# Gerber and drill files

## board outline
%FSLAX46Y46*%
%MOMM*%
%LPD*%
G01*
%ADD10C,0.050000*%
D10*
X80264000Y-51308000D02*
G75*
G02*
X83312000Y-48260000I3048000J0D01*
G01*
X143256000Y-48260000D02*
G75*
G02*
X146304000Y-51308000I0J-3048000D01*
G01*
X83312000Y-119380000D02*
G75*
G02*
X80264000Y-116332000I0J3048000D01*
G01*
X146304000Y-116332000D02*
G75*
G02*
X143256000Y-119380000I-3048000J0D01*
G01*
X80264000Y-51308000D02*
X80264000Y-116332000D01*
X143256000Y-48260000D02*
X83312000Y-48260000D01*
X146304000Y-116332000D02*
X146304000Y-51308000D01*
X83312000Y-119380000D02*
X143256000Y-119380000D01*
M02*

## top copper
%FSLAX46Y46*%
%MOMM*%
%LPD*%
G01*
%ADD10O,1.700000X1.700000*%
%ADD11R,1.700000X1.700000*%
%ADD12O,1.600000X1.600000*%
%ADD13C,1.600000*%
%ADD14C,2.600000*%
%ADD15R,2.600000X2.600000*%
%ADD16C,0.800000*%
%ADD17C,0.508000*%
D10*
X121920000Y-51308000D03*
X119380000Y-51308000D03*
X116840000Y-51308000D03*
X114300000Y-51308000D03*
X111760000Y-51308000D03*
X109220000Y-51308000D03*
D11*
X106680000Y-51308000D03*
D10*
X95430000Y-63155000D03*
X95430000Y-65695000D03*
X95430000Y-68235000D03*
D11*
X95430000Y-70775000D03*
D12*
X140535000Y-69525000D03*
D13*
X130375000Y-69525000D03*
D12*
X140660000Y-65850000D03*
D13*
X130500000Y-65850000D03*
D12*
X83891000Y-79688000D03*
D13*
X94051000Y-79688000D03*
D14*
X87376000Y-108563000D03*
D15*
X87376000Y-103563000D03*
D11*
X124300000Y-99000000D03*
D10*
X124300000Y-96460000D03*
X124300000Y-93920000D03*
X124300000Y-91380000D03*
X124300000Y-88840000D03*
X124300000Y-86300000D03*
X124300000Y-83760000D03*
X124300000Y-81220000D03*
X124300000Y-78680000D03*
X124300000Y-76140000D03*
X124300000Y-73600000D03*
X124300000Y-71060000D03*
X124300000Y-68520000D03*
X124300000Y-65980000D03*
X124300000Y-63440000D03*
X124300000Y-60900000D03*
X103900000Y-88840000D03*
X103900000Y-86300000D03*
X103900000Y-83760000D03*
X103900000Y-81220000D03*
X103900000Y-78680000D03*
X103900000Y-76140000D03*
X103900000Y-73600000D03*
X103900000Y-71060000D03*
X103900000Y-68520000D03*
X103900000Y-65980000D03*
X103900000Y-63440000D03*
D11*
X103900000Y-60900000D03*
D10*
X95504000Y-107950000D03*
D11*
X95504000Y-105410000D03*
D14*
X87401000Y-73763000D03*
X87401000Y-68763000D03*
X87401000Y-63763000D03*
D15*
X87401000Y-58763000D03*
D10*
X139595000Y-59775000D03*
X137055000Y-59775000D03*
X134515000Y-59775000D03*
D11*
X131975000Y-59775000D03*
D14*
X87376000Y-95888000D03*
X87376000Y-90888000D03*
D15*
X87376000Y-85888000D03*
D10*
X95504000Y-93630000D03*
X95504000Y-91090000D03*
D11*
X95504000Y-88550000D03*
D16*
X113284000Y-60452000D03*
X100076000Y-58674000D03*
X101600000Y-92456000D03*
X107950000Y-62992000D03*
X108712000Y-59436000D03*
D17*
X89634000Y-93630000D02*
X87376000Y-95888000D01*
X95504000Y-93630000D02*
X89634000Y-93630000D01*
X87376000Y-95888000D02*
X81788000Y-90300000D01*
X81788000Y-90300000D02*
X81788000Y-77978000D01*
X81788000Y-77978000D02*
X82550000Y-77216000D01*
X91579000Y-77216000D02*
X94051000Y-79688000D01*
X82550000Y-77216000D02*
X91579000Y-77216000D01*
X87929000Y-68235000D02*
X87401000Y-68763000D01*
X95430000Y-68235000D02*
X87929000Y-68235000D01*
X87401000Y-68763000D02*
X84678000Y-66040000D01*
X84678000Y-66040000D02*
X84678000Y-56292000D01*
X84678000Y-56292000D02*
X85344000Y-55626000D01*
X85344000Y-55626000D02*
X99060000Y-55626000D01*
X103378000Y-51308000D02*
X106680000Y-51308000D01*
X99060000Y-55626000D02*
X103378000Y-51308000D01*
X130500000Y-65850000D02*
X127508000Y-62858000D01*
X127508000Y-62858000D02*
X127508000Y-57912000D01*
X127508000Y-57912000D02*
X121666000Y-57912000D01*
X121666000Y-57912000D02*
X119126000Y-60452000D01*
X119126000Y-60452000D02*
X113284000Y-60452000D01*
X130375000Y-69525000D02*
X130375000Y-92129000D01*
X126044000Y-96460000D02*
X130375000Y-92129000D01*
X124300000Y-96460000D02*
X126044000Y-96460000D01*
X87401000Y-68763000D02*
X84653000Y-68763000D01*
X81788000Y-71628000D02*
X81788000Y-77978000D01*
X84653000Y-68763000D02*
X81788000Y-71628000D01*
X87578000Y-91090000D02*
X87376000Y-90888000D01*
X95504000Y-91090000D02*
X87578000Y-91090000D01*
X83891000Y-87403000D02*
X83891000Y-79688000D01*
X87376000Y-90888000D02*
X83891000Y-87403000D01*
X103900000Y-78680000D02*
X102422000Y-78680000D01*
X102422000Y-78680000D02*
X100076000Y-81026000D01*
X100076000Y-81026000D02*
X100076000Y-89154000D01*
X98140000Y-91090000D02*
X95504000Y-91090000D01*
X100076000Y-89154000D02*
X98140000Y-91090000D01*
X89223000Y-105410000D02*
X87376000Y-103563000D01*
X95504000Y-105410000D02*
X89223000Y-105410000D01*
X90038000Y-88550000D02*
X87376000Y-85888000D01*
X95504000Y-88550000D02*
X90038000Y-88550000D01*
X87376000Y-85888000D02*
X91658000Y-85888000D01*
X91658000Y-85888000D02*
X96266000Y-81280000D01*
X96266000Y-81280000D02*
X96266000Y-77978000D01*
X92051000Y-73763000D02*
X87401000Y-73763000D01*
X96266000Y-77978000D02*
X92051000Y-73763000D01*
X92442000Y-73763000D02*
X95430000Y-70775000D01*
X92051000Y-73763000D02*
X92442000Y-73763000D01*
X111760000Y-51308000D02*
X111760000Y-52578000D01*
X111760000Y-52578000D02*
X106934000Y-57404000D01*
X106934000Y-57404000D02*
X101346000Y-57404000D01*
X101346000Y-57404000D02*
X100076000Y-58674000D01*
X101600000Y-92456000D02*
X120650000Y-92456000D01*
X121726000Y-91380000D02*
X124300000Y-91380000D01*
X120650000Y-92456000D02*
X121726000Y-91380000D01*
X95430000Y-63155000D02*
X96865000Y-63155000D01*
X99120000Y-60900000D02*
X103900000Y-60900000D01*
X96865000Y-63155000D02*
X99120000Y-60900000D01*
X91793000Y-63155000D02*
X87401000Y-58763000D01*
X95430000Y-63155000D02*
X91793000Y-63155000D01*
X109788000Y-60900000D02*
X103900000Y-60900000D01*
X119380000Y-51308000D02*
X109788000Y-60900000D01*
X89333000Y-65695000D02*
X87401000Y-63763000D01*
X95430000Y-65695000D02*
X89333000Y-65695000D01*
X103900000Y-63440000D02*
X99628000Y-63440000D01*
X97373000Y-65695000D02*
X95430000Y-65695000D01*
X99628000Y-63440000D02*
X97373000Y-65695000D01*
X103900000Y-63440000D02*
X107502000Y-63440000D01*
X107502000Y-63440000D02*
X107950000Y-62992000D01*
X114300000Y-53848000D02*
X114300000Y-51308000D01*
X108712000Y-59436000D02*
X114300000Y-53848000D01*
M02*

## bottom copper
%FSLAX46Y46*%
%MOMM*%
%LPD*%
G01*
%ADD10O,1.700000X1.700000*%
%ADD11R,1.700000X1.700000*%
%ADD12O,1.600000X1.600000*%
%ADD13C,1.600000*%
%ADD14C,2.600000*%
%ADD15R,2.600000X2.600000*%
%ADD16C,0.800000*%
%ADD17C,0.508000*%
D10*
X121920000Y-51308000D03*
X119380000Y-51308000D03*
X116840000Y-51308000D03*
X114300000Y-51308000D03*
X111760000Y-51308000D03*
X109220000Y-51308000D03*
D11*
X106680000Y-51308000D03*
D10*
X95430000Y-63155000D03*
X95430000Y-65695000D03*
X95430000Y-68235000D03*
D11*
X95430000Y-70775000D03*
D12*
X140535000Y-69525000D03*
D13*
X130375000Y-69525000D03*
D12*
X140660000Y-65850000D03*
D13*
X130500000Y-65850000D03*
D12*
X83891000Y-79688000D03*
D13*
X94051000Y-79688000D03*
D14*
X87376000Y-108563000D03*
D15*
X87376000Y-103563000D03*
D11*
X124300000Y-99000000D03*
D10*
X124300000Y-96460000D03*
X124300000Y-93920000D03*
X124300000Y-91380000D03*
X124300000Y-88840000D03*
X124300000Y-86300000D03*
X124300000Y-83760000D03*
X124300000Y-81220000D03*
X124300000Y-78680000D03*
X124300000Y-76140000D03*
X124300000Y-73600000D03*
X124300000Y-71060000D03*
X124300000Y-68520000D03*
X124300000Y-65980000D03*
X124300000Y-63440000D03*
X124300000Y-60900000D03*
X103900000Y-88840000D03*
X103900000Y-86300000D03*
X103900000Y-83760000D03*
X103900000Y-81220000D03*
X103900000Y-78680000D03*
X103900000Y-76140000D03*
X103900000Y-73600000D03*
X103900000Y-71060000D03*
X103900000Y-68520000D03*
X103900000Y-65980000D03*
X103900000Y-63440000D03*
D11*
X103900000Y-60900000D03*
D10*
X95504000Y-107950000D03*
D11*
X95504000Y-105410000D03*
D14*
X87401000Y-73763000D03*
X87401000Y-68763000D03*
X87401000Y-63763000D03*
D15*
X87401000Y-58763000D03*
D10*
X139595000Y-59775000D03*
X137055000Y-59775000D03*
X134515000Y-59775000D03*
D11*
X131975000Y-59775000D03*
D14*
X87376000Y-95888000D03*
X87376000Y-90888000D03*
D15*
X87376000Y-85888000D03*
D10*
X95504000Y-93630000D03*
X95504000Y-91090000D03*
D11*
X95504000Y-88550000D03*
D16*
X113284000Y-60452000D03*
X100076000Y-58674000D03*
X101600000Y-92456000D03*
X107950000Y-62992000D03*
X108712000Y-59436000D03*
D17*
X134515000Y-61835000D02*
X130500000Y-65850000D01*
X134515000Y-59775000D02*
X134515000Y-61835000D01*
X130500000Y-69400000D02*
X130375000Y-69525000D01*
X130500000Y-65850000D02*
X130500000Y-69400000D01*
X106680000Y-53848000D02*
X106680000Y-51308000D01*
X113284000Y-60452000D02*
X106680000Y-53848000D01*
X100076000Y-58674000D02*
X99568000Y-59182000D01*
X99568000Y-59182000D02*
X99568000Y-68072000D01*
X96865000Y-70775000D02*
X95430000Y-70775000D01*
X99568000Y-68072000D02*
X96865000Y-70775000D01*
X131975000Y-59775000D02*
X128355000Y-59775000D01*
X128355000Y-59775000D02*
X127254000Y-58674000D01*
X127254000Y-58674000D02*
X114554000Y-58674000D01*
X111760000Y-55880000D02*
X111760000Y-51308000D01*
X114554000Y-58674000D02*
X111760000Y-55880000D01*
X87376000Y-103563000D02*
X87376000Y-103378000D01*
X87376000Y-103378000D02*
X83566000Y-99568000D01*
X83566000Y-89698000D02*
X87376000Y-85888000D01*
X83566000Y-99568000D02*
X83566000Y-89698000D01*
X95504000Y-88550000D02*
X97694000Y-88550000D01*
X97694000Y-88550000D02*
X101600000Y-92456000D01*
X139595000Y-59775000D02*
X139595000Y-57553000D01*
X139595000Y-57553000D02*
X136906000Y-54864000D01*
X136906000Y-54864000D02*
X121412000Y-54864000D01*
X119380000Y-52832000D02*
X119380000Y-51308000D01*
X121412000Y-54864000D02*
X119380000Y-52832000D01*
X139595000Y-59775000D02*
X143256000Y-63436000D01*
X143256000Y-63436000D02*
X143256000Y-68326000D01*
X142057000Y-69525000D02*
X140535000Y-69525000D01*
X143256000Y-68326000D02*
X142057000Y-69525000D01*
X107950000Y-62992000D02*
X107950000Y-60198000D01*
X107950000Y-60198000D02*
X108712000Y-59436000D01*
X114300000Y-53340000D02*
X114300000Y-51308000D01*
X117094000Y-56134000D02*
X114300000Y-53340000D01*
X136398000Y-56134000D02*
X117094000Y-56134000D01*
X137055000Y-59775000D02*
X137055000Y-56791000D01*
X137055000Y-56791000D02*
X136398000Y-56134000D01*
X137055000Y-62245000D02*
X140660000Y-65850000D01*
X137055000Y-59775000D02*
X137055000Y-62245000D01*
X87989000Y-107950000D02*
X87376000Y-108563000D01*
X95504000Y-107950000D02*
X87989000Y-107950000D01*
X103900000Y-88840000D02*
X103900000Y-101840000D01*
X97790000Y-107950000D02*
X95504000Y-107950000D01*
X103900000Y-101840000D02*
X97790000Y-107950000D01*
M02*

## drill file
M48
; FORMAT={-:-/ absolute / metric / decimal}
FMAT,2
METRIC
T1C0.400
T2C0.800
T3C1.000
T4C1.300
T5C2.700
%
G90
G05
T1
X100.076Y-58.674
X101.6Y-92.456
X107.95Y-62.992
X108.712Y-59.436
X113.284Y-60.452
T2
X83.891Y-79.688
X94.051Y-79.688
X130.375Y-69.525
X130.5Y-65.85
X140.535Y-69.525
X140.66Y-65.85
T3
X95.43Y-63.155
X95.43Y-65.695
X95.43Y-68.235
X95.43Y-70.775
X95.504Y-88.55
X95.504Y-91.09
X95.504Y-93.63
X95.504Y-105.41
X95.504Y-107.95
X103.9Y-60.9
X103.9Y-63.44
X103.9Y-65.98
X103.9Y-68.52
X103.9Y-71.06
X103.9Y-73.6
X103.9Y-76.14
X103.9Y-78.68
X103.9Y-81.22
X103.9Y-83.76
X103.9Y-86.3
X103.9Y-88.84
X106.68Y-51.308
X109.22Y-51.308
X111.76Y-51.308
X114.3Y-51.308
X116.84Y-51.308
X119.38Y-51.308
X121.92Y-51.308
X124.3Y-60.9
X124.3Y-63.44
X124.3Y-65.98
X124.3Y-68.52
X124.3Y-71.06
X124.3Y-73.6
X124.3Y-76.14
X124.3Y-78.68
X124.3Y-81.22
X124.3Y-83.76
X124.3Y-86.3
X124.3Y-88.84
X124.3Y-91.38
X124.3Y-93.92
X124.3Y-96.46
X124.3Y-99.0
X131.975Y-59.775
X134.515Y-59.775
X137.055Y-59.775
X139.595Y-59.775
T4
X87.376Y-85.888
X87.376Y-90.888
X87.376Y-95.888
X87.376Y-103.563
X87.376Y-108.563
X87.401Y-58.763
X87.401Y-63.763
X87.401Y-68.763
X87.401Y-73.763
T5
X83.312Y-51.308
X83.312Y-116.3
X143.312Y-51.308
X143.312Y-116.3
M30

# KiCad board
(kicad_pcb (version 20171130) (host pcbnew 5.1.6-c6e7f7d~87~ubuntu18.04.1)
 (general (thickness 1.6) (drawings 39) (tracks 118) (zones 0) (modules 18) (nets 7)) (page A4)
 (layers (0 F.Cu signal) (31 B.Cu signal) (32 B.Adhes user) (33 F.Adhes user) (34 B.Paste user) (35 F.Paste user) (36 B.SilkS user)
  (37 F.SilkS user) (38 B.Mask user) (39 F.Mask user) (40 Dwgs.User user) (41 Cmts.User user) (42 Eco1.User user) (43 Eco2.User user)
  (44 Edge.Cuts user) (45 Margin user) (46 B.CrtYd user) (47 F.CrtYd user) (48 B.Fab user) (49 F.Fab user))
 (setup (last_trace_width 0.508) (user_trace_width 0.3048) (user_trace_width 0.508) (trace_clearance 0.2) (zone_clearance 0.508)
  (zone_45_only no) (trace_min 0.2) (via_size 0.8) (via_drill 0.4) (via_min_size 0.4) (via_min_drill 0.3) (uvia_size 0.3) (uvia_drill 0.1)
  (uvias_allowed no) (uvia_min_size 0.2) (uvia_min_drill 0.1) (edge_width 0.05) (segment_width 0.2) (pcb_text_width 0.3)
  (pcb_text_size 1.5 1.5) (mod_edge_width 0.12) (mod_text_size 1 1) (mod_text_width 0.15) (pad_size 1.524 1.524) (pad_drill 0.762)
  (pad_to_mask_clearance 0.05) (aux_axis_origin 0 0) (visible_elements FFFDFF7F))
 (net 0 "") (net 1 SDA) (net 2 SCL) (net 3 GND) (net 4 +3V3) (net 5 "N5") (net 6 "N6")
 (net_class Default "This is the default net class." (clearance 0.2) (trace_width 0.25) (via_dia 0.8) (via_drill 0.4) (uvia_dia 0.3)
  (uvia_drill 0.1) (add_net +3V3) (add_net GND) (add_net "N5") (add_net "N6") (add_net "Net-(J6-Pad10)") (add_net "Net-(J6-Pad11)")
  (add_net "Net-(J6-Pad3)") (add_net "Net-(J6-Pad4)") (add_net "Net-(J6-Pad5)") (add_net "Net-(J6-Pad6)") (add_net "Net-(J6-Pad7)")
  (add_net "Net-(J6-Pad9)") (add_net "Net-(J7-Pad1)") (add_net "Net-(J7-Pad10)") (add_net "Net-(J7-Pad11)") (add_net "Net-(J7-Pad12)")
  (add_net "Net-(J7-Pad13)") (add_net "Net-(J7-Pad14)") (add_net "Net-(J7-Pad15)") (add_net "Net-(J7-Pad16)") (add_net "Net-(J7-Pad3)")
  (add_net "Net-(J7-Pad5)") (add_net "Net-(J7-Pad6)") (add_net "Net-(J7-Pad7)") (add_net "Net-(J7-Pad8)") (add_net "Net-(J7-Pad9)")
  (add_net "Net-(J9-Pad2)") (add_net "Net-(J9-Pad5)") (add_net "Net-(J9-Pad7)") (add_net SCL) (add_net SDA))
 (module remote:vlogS (layer F.Cu) (at 136.652 107.442)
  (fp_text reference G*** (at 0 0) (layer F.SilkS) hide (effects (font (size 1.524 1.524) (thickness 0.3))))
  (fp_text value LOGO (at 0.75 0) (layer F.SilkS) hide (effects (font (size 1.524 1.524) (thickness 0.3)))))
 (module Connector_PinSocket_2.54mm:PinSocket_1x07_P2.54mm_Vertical (layer F.Cu) (at 106.68 51.308 90)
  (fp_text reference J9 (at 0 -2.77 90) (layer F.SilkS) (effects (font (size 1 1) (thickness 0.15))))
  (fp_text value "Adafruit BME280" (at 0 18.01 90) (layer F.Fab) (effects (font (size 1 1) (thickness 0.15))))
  (pad 7 thru_hole oval (at 0 15.24 90) (size 1.7 1.7) (drill 1) (layers *.Cu *.Mask))
  (pad 6 thru_hole oval (at 0 12.7 90) (size 1.7 1.7) (drill 1) (layers *.Cu *.Mask) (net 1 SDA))
  (pad 5 thru_hole oval (at 0 10.16 90) (size 1.7 1.7) (drill 1) (layers *.Cu *.Mask))
  (pad 4 thru_hole oval (at 0 7.62 90) (size 1.7 1.7) (drill 1) (layers *.Cu *.Mask) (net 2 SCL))
  (pad 3 thru_hole oval (at 0 5.08 90) (size 1.7 1.7) (drill 1) (layers *.Cu *.Mask) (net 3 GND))
  (pad 2 thru_hole oval (at 0 2.54 90) (size 1.7 1.7) (drill 1) (layers *.Cu *.Mask))
  (pad 1 thru_hole rect (at 0 0 90) (size 1.7 1.7) (drill 1) (layers *.Cu *.Mask) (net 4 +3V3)))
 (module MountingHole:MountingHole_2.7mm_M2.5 (layer F.Cu) (at 143.312 116.3)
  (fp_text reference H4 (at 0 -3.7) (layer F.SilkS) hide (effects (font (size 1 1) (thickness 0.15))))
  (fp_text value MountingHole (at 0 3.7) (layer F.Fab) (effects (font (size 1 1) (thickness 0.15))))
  (pad 1 np_thru_hole circle (at 0 0) (size 2.7 2.7) (drill 2.7) (layers *.Cu *.Mask)))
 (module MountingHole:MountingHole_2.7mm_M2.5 (layer F.Cu) (at 83.312 116.3)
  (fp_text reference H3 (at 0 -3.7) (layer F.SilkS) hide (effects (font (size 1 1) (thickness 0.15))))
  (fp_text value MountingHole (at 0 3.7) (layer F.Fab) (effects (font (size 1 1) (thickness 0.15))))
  (pad 1 np_thru_hole circle (at 0 0) (size 2.7 2.7) (drill 2.7) (layers *.Cu *.Mask)))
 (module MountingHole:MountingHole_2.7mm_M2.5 (layer F.Cu) (at 143.312 51.308)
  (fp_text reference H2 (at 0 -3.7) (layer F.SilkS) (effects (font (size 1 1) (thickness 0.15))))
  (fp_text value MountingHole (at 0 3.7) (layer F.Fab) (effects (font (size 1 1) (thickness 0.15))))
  (pad 1 np_thru_hole circle (at 0 0) (size 2.7 2.7) (drill 2.7) (layers *.Cu *.Mask)))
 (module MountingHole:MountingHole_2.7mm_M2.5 (layer F.Cu) (at 83.312 51.308)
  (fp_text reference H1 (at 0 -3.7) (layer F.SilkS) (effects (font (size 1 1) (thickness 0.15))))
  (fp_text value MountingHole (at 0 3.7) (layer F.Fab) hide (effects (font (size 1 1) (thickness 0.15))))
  (pad 1 np_thru_hole circle (at 0 0) (size 2.7 2.7) (drill 2.7) (layers *.Cu *.Mask)))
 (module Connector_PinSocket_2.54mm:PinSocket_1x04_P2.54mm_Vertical (layer F.Cu) (at 95.43 70.775 180)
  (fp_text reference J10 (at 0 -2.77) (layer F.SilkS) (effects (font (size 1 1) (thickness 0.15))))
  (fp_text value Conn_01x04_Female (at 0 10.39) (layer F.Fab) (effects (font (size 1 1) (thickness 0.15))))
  (pad 4 thru_hole oval (at 0 7.62 180) (size 1.7 1.7) (drill 1) (layers *.Cu *.Mask) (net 1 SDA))
  (pad 3 thru_hole oval (at 0 5.08 180) (size 1.7 1.7) (drill 1) (layers *.Cu *.Mask) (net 2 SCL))
  (pad 2 thru_hole oval (at 0 2.54 180) (size 1.7 1.7) (drill 1) (layers *.Cu *.Mask) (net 4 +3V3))
  (pad 1 thru_hole rect (at 0 0 180) (size 1.7 1.7) (drill 1) (layers *.Cu *.Mask) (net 3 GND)))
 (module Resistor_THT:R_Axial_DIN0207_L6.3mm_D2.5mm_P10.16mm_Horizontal (layer F.Cu) (at 130.375 69.525)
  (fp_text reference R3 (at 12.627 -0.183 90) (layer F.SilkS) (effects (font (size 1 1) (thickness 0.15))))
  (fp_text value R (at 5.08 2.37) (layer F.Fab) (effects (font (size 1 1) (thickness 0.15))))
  (pad 2 thru_hole oval (at 10.16 0) (size 1.6 1.6) (drill 0.8) (layers *.Cu *.Mask) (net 1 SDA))
  (pad 1 thru_hole circle (at 0 0) (size 1.6 1.6) (drill 0.8) (layers *.Cu *.Mask) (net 4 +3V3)))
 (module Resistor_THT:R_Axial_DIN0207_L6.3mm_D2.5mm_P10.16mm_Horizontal (layer F.Cu) (at 130.5 65.85)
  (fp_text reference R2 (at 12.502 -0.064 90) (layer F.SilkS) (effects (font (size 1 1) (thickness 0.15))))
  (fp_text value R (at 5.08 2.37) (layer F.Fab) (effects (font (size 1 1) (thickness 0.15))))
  (pad 2 thru_hole oval (at 10.16 0) (size 1.6 1.6) (drill 0.8) (layers *.Cu *.Mask) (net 2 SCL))
  (pad 1 thru_hole circle (at 0 0) (size 1.6 1.6) (drill 0.8) (layers *.Cu *.Mask) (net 4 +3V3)))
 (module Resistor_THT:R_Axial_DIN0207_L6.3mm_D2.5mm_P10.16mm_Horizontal (layer F.Cu) (at 94.051 79.688 180)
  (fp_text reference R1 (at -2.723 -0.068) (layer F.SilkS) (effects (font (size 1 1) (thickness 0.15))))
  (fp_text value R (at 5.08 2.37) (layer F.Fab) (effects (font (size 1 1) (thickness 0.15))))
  (pad 2 thru_hole oval (at 10.16 0 180) (size 1.6 1.6) (drill 0.8) (layers *.Cu *.Mask) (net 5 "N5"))
  (pad 1 thru_hole circle (at 0 0 180) (size 1.6 1.6) (drill 0.8) (layers *.Cu *.Mask) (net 4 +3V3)))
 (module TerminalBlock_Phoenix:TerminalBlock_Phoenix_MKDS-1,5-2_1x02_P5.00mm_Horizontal (layer F.Cu) (at 87.376 103.563 270)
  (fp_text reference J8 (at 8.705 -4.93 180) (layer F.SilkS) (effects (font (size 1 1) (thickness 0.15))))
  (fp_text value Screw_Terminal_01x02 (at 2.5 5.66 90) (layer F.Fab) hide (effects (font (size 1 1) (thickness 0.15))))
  (pad 2 thru_hole circle (at 5 0 270) (size 2.6 2.6) (drill 1.3) (layers *.Cu *.Mask) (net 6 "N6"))
  (pad 1 thru_hole rect (at 0 0 270) (size 2.6 2.6) (drill 1.3) (layers *.Cu *.Mask) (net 3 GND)))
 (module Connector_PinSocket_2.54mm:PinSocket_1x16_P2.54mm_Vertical (layer F.Cu) (at 124.3 99 180)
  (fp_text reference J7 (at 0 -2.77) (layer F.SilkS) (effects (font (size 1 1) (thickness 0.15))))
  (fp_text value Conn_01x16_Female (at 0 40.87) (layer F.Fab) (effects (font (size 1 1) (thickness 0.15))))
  (pad 1 thru_hole rect (at 0 0 180) (size 1.7 1.7) (drill 1) (layers *.Cu *.Mask))
  (pad 2 thru_hole oval (at 0 2.54 180) (size 1.7 1.7) (drill 1) (layers *.Cu *.Mask) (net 4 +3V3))
  (pad 3 thru_hole oval (at 0 5.08 180) (size 1.7 1.7) (drill 1) (layers *.Cu *.Mask))
  (pad 4 thru_hole oval (at 0 7.62 180) (size 1.7 1.7) (drill 1) (layers *.Cu *.Mask) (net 3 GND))
  (pad 5 thru_hole oval (at 0 10.16 180) (size 1.7 1.7) (drill 1) (layers *.Cu *.Mask))
  (pad 6 thru_hole oval (at 0 12.7 180) (size 1.7 1.7) (drill 1) (layers *.Cu *.Mask))
  (pad 7 thru_hole oval (at 0 15.24 180) (size 1.7 1.7) (drill 1) (layers *.Cu *.Mask))
  (pad 8 thru_hole oval (at 0 17.78 180) (size 1.7 1.7) (drill 1) (layers *.Cu *.Mask))
  (pad 9 thru_hole oval (at 0 20.32 180) (size 1.7 1.7) (drill 1) (layers *.Cu *.Mask))
  (pad 10 thru_hole oval (at 0 22.86 180) (size 1.7 1.7) (drill 1) (layers *.Cu *.Mask))
  (pad 11 thru_hole oval (at 0 25.4 180) (size 1.7 1.7) (drill 1) (layers *.Cu *.Mask))
  (pad 12 thru_hole oval (at 0 27.94 180) (size 1.7 1.7) (drill 1) (layers *.Cu *.Mask))
  (pad 13 thru_hole oval (at 0 30.48 180) (size 1.7 1.7) (drill 1) (layers *.Cu *.Mask))
  (pad 14 thru_hole oval (at 0 33.02 180) (size 1.7 1.7) (drill 1) (layers *.Cu *.Mask))
  (pad 15 thru_hole oval (at 0 35.56 180) (size 1.7 1.7) (drill 1) (layers *.Cu *.Mask))
  (pad 16 thru_hole oval (at 0 38.1 180) (size 1.7 1.7) (drill 1) (layers *.Cu *.Mask)))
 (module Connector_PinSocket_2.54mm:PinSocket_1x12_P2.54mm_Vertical (layer F.Cu) (at 103.9 60.9)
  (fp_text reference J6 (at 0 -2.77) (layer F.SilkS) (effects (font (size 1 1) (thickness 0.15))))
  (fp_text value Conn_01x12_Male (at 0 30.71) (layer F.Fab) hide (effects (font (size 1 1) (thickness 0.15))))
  (pad 12 thru_hole oval (at 0 27.94) (size 1.7 1.7) (drill 1) (layers *.Cu *.Mask) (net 6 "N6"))
  (pad 11 thru_hole oval (at 0 25.4) (size 1.7 1.7) (drill 1) (layers *.Cu *.Mask))
  (pad 10 thru_hole oval (at 0 22.86) (size 1.7 1.7) (drill 1) (layers *.Cu *.Mask))
  (pad 9 thru_hole oval (at 0 20.32) (size 1.7 1.7) (drill 1) (layers *.Cu *.Mask))
  (pad 8 thru_hole oval (at 0 17.78) (size 1.7 1.7) (drill 1) (layers *.Cu *.Mask) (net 5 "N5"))
  (pad 7 thru_hole oval (at 0 15.24) (size 1.7 1.7) (drill 1) (layers *.Cu *.Mask))
  (pad 6 thru_hole oval (at 0 12.7) (size 1.7 1.7) (drill 1) (layers *.Cu *.Mask))
  (pad 5 thru_hole oval (at 0 10.16) (size 1.7 1.7) (drill 1) (layers *.Cu *.Mask))
  (pad 4 thru_hole oval (at 0 7.62) (size 1.7 1.7) (drill 1) (layers *.Cu *.Mask))
  (pad 3 thru_hole oval (at 0 5.08) (size 1.7 1.7) (drill 1) (layers *.Cu *.Mask))
  (pad 2 thru_hole oval (at 0 2.54) (size 1.7 1.7) (drill 1) (layers *.Cu *.Mask) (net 2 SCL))
  (pad 1 thru_hole rect (at 0 0) (size 1.7 1.7) (drill 1) (layers *.Cu *.Mask) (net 1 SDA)))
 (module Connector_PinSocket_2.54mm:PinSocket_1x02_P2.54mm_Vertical (layer F.Cu) (at 95.504 105.41)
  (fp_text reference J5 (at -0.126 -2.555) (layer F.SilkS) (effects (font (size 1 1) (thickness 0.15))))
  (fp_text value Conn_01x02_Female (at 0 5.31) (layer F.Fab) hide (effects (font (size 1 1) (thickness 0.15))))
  (pad 2 thru_hole oval (at 0 2.54) (size 1.7 1.7) (drill 1) (layers *.Cu *.Mask) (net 6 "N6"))
  (pad 1 thru_hole rect (at 0 0) (size 1.7 1.7) (drill 1) (layers *.Cu *.Mask) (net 3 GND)))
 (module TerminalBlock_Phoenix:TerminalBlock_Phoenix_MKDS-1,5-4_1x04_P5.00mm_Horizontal (layer F.Cu) (at 87.401 58.763 270)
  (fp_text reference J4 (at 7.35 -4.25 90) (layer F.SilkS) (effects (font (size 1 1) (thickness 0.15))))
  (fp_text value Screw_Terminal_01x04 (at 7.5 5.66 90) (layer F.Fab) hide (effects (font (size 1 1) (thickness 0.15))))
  (pad 4 thru_hole circle (at 15 0 270) (size 2.6 2.6) (drill 1.3) (layers *.Cu *.Mask) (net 3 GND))
  (pad 3 thru_hole circle (at 10 0 270) (size 2.6 2.6) (drill 1.3) (layers *.Cu *.Mask) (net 4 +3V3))
  (pad 2 thru_hole circle (at 5 0 270) (size 2.6 2.6) (drill 1.3) (layers *.Cu *.Mask) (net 2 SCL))
  (pad 1 thru_hole rect (at 0 0 270) (size 2.6 2.6) (drill 1.3) (layers *.Cu *.Mask) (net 1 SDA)))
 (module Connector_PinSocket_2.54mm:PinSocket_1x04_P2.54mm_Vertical (layer F.Cu) (at 131.975 59.775 90)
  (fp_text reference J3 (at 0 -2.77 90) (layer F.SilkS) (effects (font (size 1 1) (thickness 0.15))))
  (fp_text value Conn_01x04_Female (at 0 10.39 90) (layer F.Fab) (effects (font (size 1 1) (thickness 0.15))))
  (pad 4 thru_hole oval (at 0 7.62 90) (size 1.7 1.7) (drill 1) (layers *.Cu *.Mask) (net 1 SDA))
  (pad 3 thru_hole oval (at 0 5.08 90) (size 1.7 1.7) (drill 1) (layers *.Cu *.Mask) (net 2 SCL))
  (pad 2 thru_hole oval (at 0 2.54 90) (size 1.7 1.7) (drill 1) (layers *.Cu *.Mask) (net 4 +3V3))
  (pad 1 thru_hole rect (at 0 0 90) (size 1.7 1.7) (drill 1) (layers *.Cu *.Mask) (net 3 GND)))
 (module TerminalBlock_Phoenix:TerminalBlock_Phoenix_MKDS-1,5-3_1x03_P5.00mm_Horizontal (layer F.Cu) (at 87.376 85.888 270)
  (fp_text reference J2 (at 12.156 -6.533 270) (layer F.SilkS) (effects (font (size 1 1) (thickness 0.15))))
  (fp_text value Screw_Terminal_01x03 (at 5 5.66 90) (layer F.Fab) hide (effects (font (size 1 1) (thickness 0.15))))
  (pad 3 thru_hole circle (at 10 0 270) (size 2.6 2.6) (drill 1.3) (layers *.Cu *.Mask) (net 4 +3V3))
  (pad 2 thru_hole circle (at 5 0 270) (size 2.6 2.6) (drill 1.3) (layers *.Cu *.Mask) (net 5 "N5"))
  (pad 1 thru_hole rect (at 0 0 270) (size 2.6 2.6) (drill 1.3) (layers *.Cu *.Mask) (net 3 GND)))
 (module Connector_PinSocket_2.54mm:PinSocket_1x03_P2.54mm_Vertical (layer F.Cu) (at 95.504 88.55)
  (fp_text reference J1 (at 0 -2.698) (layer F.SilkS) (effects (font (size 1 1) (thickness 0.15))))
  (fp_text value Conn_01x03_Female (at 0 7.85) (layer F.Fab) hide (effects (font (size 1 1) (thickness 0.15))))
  (pad 3 thru_hole oval (at 0 5.08) (size 1.7 1.7) (drill 1) (layers *.Cu *.Mask) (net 4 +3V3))
  (pad 2 thru_hole oval (at 0 2.54) (size 1.7 1.7) (drill 1) (layers *.Cu *.Mask) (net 5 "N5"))
  (pad 1 thru_hole rect (at 0 0) (size 1.7 1.7) (drill 1) (layers *.Cu *.Mask) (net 3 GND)))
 (gr_arc (start 83.312 51.308) (end 83.312 48.26) (angle -90) (layer Edge.Cuts) (width 0.05))
 (gr_arc (start 143.256 51.308) (end 146.304 51.308) (angle -90) (layer Edge.Cuts) (width 0.05))
 (gr_arc (start 83.312 116.332) (end 80.264 116.332) (angle -90) (layer Edge.Cuts) (width 0.05))
 (gr_arc (start 143.256 116.332) (end 143.256 119.38) (angle -90) (layer Edge.Cuts) (width 0.05))
 (gr_line (start 80.264 51.308) (end 80.264 116.332) (layer Edge.Cuts) (width 0.05))
 (gr_line (start 143.256 48.26) (end 83.312 48.26) (layer Edge.Cuts) (width 0.05))
 (gr_line (start 146.304 116.332) (end 146.304 51.308) (layer Edge.Cuts) (width 0.05))
 (gr_line (start 83.312 119.38) (end 143.256 119.38) (layer Edge.Cuts) (width 0.05))
 (segment (start 89.634 93.63) (end 87.376 95.888) (width 0.508) (layer F.Cu) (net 4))
 (segment (start 95.504 93.63) (end 89.634 93.63) (width 0.508) (layer F.Cu) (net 4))
 (segment (start 87.376 95.888) (end 81.788 90.3) (width 0.508) (layer F.Cu) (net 4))
 (segment (start 81.788 90.3) (end 81.788 77.978) (width 0.508) (layer F.Cu) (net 4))
 (segment (start 81.788 77.978) (end 82.55 77.216) (width 0.508) (layer F.Cu) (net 4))
 (segment (start 91.579 77.216) (end 94.051 79.688) (width 0.508) (layer F.Cu) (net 4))
 (segment (start 82.55 77.216) (end 91.579 77.216) (width 0.508) (layer F.Cu) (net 4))
 (segment (start 87.929 68.235) (end 87.401 68.763) (width 0.508) (layer F.Cu) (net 4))
 (segment (start 95.43 68.235) (end 87.929 68.235) (width 0.508) (layer F.Cu) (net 4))
 (segment (start 87.401 68.763) (end 84.678 66.04) (width 0.508) (layer F.Cu) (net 4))
 (segment (start 84.678 66.04) (end 84.678 56.292) (width 0.508) (layer F.Cu) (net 4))
 (segment (start 84.678 56.292) (end 85.344 55.626) (width 0.508) (layer F.Cu) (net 4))
 (segment (start 85.344 55.626) (end 99.06 55.626) (width 0.508) (layer F.Cu) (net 4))
 (segment (start 103.378 51.308) (end 106.68 51.308) (width 0.508) (layer F.Cu) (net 4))
 (segment (start 99.06 55.626) (end 103.378 51.308) (width 0.508) (layer F.Cu) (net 4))
 (segment (start 134.515 61.835) (end 130.5 65.85) (width 0.508) (layer B.Cu) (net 4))
 (segment (start 134.515 59.775) (end 134.515 61.835) (width 0.508) (layer B.Cu) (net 4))
 (segment (start 130.5 69.4) (end 130.375 69.525) (width 0.508) (layer B.Cu) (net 4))
 (segment (start 130.5 65.85) (end 130.5 69.4) (width 0.508) (layer B.Cu) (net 4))
 (segment (start 130.5 65.85) (end 127.508 62.858) (width 0.508) (layer F.Cu) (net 4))
 (segment (start 127.508 62.858) (end 127.508 57.912) (width 0.508) (layer F.Cu) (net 4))
 (segment (start 127.508 57.912) (end 121.666 57.912) (width 0.508) (layer F.Cu) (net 4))
 (via (at 113.284 60.452) (size 0.8) (drill 0.4) (layers F.Cu B.Cu) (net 4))
 (segment (start 121.666 57.912) (end 119.126 60.452) (width 0.508) (layer F.Cu) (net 4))
 (segment (start 119.126 60.452) (end 113.284 60.452) (width 0.508) (layer F.Cu) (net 4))
 (segment (start 106.68 53.848) (end 106.68 51.308) (width 0.508) (layer B.Cu) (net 4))
 (segment (start 113.284 60.452) (end 106.68 53.848) (width 0.508) (layer B.Cu) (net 4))
 (segment (start 130.375 69.525) (end 130.375 92.129) (width 0.508) (layer F.Cu) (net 4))
 (segment (start 126.044 96.46) (end 130.375 92.129) (width 0.508) (layer F.Cu) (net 4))
 (segment (start 124.3 96.46) (end 126.044 96.46) (width 0.508) (layer F.Cu) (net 4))
 (segment (start 87.401 68.763) (end 84.653 68.763) (width 0.508) (layer F.Cu) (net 4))
 (segment (start 81.788 71.628) (end 81.788 77.978) (width 0.508) (layer F.Cu) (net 4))
 (segment (start 84.653 68.763) (end 81.788 71.628) (width 0.508) (layer F.Cu) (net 4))
 (segment (start 87.578 91.09) (end 87.376 90.888) (width 0.508) (layer F.Cu) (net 5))
 (segment (start 95.504 91.09) (end 87.578 91.09) (width 0.508) (layer F.Cu) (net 5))
 (segment (start 83.891 87.403) (end 83.891 79.688) (width 0.508) (layer F.Cu) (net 5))
 (segment (start 87.376 90.888) (end 83.891 87.403) (width 0.508) (layer F.Cu) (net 5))
 (segment (start 103.9 78.68) (end 102.422 78.68) (width 0.508) (layer F.Cu) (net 5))
 (segment (start 102.422 78.68) (end 100.076 81.026) (width 0.508) (layer F.Cu) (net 5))
 (segment (start 100.076 81.026) (end 100.076 89.154) (width 0.508) (layer F.Cu) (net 5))
 (segment (start 98.14 91.09) (end 95.504 91.09) (width 0.508) (layer F.Cu) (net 5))
 (segment (start 100.076 89.154) (end 98.14 91.09) (width 0.508) (layer F.Cu) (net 5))
 (segment (start 89.223 105.41) (end 87.376 103.563) (width 0.508) (layer F.Cu) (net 3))
 (segment (start 95.504 105.41) (end 89.223 105.41) (width 0.508) (layer F.Cu) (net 3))
 (segment (start 90.038 88.55) (end 87.376 85.888) (width 0.508) (layer F.Cu) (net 3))
 (segment (start 95.504 88.55) (end 90.038 88.55) (width 0.508) (layer F.Cu) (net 3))
 (segment (start 87.376 85.888) (end 91.658 85.888) (width 0.508) (layer F.Cu) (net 3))
 (segment (start 91.658 85.888) (end 96.266 81.28) (width 0.508) (layer F.Cu) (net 3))
 (segment (start 96.266 81.28) (end 96.266 77.978) (width 0.508) (layer F.Cu) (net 3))
 (segment (start 92.051 73.763) (end 87.401 73.763) (width 0.508) (layer F.Cu) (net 3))
 (segment (start 96.266 77.978) (end 92.051 73.763) (width 0.508) (layer F.Cu) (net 3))
 (segment (start 92.442 73.763) (end 95.43 70.775) (width 0.508) (layer F.Cu) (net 3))
 (segment (start 92.051 73.763) (end 92.442 73.763) (width 0.508) (layer F.Cu) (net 3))
 (segment (start 111.76 51.308) (end 111.76 52.578) (width 0.508) (layer F.Cu) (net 3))
 (segment (start 111.76 52.578) (end 106.934 57.404) (width 0.508) (layer F.Cu) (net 3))
 (via (at 100.076 58.674) (size 0.8) (drill 0.4) (layers F.Cu B.Cu) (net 3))
 (segment (start 106.934 57.404) (end 101.346 57.404) (width 0.508) (layer F.Cu) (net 3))
 (segment (start 101.346 57.404) (end 100.076 58.674) (width 0.508) (layer F.Cu) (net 3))
 (segment (start 100.076 58.674) (end 99.568 59.182) (width 0.508) (layer B.Cu) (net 3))
 (segment (start 99.568 59.182) (end 99.568 68.072) (width 0.508) (layer B.Cu) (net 3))
 (segment (start 96.865 70.775) (end 95.43 70.775) (width 0.508) (layer B.Cu) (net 3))
 (segment (start 99.568 68.072) (end 96.865 70.775) (width 0.508) (layer B.Cu) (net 3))
 (segment (start 131.975 59.775) (end 128.355 59.775) (width 0.508) (layer B.Cu) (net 3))
 (segment (start 128.355 59.775) (end 127.254 58.674) (width 0.508) (layer B.Cu) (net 3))
 (segment (start 127.254 58.674) (end 114.554 58.674) (width 0.508) (layer B.Cu) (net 3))
 (segment (start 111.76 55.88) (end 111.76 51.308) (width 0.508) (layer B.Cu) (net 3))
 (segment (start 114.554 58.674) (end 111.76 55.88) (width 0.508) (layer B.Cu) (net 3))
 (segment (start 87.376 103.563) (end 87.376 103.378) (width 0.508) (layer B.Cu) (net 3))
 (segment (start 87.376 103.378) (end 83.566 99.568) (width 0.508) (layer B.Cu) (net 3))
 (segment (start 83.566 89.698) (end 87.376 85.888) (width 0.508) (layer B.Cu) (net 3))
 (segment (start 83.566 99.568) (end 83.566 89.698) (width 0.508) (layer B.Cu) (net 3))
 (segment (start 95.504 88.55) (end 97.694 88.55) (width 0.508) (layer B.Cu) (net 3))
 (segment (start 97.694 88.55) (end 101.6 92.456) (width 0.508) (layer B.Cu) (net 3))
 (via (at 101.6 92.456) (size 0.8) (drill 0.4) (layers F.Cu B.Cu) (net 3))
 (segment (start 101.6 92.456) (end 120.65 92.456) (width 0.508) (layer F.Cu) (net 3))
 (segment (start 121.726 91.38) (end 124.3 91.38) (width 0.508) (layer F.Cu) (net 3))
 (segment (start 120.65 92.456) (end 121.726 91.38) (width 0.508) (layer F.Cu) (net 3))
 (segment (start 95.43 63.155) (end 96.865 63.155) (width 0.508) (layer F.Cu) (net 1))
 (segment (start 99.12 60.9) (end 103.9 60.9) (width 0.508) (layer F.Cu) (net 1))
 (segment (start 96.865 63.155) (end 99.12 60.9) (width 0.508) (layer F.Cu) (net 1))
 (segment (start 91.793 63.155) (end 87.401 58.763) (width 0.508) (layer F.Cu) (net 1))
 (segment (start 95.43 63.155) (end 91.793 63.155) (width 0.508) (layer F.Cu) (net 1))
 (segment (start 109.788 60.9) (end 103.9 60.9) (width 0.508) (layer F.Cu) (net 1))
 (segment (start 119.38 51.308) (end 109.788 60.9) (width 0.508) (layer F.Cu) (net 1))
 (segment (start 139.595 59.775) (end 139.595 57.553) (width 0.508) (layer B.Cu) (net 1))
 (segment (start 139.595 57.553) (end 136.906 54.864) (width 0.508) (layer B.Cu) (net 1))
 (segment (start 136.906 54.864) (end 121.412 54.864) (width 0.508) (layer B.Cu) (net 1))
 (segment (start 119.38 52.832) (end 119.38 51.308) (width 0.508) (layer B.Cu) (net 1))
 (segment (start 121.412 54.864) (end 119.38 52.832) (width 0.508) (layer B.Cu) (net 1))
 (segment (start 139.595 59.775) (end 143.256 63.436) (width 0.508) (layer B.Cu) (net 1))
 (segment (start 143.256 63.436) (end 143.256 68.326) (width 0.508) (layer B.Cu) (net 1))
 (segment (start 142.057 69.525) (end 140.535 69.525) (width 0.508) (layer B.Cu) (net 1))
 (segment (start 143.256 68.326) (end 142.057 69.525) (width 0.508) (layer B.Cu) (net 1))
 (segment (start 89.333 65.695) (end 87.401 63.763) (width 0.508) (layer F.Cu) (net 2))
 (segment (start 95.43 65.695) (end 89.333 65.695) (width 0.508) (layer F.Cu) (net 2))
 (segment (start 103.9 63.44) (end 99.628 63.44) (width 0.508) (layer F.Cu) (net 2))
 (segment (start 97.373 65.695) (end 95.43 65.695) (width 0.508) (layer F.Cu) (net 2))
 (segment (start 99.628 63.44) (end 97.373 65.695) (width 0.508) (layer F.Cu) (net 2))
 (via (at 107.95 62.992) (size 0.8) (drill 0.4) (layers F.Cu B.Cu) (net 2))
 (segment (start 103.9 63.44) (end 107.502 63.44) (width 0.508) (layer F.Cu) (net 2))
 (segment (start 107.502 63.44) (end 107.95 62.992) (width 0.508) (layer F.Cu) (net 2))
 (via (at 108.712 59.436) (size 0.8) (drill 0.4) (layers F.Cu B.Cu) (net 2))
 (segment (start 107.95 62.992) (end 107.95 60.198) (width 0.508) (layer B.Cu) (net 2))
 (segment (start 107.95 60.198) (end 108.712 59.436) (width 0.508) (layer B.Cu) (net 2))
 (segment (start 114.3 53.848) (end 114.3 51.308) (width 0.508) (layer F.Cu) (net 2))
 (segment (start 108.712 59.436) (end 114.3 53.848) (width 0.508) (layer F.Cu) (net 2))
 (segment (start 114.3 53.34) (end 114.3 51.308) (width 0.508) (layer B.Cu) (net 2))
 (segment (start 117.094 56.134) (end 114.3 53.34) (width 0.508) (layer B.Cu) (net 2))
 (segment (start 136.398 56.134) (end 117.094 56.134) (width 0.508) (layer B.Cu) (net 2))
 (segment (start 137.055 59.775) (end 137.055 56.791) (width 0.508) (layer B.Cu) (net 2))
 (segment (start 137.055 56.791) (end 136.398 56.134) (width 0.508) (layer B.Cu) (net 2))
 (segment (start 137.055 62.245) (end 140.66 65.85) (width 0.508) (layer B.Cu) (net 2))
 (segment (start 137.055 59.775) (end 137.055 62.245) (width 0.508) (layer B.Cu) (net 2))
 (segment (start 87.989 107.95) (end 87.376 108.563) (width 0.508) (layer B.Cu) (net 6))
 (segment (start 95.504 107.95) (end 87.989 107.95) (width 0.508) (layer B.Cu) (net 6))
 (segment (start 103.9 88.84) (end 103.9 101.84) (width 0.508) (layer B.Cu) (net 6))
 (segment (start 97.79 107.95) (end 95.504 107.95) (width 0.508) (layer B.Cu) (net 6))
 (segment (start 103.9 101.84) (end 97.79 107.95) (width 0.508) (layer B.Cu) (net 6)))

